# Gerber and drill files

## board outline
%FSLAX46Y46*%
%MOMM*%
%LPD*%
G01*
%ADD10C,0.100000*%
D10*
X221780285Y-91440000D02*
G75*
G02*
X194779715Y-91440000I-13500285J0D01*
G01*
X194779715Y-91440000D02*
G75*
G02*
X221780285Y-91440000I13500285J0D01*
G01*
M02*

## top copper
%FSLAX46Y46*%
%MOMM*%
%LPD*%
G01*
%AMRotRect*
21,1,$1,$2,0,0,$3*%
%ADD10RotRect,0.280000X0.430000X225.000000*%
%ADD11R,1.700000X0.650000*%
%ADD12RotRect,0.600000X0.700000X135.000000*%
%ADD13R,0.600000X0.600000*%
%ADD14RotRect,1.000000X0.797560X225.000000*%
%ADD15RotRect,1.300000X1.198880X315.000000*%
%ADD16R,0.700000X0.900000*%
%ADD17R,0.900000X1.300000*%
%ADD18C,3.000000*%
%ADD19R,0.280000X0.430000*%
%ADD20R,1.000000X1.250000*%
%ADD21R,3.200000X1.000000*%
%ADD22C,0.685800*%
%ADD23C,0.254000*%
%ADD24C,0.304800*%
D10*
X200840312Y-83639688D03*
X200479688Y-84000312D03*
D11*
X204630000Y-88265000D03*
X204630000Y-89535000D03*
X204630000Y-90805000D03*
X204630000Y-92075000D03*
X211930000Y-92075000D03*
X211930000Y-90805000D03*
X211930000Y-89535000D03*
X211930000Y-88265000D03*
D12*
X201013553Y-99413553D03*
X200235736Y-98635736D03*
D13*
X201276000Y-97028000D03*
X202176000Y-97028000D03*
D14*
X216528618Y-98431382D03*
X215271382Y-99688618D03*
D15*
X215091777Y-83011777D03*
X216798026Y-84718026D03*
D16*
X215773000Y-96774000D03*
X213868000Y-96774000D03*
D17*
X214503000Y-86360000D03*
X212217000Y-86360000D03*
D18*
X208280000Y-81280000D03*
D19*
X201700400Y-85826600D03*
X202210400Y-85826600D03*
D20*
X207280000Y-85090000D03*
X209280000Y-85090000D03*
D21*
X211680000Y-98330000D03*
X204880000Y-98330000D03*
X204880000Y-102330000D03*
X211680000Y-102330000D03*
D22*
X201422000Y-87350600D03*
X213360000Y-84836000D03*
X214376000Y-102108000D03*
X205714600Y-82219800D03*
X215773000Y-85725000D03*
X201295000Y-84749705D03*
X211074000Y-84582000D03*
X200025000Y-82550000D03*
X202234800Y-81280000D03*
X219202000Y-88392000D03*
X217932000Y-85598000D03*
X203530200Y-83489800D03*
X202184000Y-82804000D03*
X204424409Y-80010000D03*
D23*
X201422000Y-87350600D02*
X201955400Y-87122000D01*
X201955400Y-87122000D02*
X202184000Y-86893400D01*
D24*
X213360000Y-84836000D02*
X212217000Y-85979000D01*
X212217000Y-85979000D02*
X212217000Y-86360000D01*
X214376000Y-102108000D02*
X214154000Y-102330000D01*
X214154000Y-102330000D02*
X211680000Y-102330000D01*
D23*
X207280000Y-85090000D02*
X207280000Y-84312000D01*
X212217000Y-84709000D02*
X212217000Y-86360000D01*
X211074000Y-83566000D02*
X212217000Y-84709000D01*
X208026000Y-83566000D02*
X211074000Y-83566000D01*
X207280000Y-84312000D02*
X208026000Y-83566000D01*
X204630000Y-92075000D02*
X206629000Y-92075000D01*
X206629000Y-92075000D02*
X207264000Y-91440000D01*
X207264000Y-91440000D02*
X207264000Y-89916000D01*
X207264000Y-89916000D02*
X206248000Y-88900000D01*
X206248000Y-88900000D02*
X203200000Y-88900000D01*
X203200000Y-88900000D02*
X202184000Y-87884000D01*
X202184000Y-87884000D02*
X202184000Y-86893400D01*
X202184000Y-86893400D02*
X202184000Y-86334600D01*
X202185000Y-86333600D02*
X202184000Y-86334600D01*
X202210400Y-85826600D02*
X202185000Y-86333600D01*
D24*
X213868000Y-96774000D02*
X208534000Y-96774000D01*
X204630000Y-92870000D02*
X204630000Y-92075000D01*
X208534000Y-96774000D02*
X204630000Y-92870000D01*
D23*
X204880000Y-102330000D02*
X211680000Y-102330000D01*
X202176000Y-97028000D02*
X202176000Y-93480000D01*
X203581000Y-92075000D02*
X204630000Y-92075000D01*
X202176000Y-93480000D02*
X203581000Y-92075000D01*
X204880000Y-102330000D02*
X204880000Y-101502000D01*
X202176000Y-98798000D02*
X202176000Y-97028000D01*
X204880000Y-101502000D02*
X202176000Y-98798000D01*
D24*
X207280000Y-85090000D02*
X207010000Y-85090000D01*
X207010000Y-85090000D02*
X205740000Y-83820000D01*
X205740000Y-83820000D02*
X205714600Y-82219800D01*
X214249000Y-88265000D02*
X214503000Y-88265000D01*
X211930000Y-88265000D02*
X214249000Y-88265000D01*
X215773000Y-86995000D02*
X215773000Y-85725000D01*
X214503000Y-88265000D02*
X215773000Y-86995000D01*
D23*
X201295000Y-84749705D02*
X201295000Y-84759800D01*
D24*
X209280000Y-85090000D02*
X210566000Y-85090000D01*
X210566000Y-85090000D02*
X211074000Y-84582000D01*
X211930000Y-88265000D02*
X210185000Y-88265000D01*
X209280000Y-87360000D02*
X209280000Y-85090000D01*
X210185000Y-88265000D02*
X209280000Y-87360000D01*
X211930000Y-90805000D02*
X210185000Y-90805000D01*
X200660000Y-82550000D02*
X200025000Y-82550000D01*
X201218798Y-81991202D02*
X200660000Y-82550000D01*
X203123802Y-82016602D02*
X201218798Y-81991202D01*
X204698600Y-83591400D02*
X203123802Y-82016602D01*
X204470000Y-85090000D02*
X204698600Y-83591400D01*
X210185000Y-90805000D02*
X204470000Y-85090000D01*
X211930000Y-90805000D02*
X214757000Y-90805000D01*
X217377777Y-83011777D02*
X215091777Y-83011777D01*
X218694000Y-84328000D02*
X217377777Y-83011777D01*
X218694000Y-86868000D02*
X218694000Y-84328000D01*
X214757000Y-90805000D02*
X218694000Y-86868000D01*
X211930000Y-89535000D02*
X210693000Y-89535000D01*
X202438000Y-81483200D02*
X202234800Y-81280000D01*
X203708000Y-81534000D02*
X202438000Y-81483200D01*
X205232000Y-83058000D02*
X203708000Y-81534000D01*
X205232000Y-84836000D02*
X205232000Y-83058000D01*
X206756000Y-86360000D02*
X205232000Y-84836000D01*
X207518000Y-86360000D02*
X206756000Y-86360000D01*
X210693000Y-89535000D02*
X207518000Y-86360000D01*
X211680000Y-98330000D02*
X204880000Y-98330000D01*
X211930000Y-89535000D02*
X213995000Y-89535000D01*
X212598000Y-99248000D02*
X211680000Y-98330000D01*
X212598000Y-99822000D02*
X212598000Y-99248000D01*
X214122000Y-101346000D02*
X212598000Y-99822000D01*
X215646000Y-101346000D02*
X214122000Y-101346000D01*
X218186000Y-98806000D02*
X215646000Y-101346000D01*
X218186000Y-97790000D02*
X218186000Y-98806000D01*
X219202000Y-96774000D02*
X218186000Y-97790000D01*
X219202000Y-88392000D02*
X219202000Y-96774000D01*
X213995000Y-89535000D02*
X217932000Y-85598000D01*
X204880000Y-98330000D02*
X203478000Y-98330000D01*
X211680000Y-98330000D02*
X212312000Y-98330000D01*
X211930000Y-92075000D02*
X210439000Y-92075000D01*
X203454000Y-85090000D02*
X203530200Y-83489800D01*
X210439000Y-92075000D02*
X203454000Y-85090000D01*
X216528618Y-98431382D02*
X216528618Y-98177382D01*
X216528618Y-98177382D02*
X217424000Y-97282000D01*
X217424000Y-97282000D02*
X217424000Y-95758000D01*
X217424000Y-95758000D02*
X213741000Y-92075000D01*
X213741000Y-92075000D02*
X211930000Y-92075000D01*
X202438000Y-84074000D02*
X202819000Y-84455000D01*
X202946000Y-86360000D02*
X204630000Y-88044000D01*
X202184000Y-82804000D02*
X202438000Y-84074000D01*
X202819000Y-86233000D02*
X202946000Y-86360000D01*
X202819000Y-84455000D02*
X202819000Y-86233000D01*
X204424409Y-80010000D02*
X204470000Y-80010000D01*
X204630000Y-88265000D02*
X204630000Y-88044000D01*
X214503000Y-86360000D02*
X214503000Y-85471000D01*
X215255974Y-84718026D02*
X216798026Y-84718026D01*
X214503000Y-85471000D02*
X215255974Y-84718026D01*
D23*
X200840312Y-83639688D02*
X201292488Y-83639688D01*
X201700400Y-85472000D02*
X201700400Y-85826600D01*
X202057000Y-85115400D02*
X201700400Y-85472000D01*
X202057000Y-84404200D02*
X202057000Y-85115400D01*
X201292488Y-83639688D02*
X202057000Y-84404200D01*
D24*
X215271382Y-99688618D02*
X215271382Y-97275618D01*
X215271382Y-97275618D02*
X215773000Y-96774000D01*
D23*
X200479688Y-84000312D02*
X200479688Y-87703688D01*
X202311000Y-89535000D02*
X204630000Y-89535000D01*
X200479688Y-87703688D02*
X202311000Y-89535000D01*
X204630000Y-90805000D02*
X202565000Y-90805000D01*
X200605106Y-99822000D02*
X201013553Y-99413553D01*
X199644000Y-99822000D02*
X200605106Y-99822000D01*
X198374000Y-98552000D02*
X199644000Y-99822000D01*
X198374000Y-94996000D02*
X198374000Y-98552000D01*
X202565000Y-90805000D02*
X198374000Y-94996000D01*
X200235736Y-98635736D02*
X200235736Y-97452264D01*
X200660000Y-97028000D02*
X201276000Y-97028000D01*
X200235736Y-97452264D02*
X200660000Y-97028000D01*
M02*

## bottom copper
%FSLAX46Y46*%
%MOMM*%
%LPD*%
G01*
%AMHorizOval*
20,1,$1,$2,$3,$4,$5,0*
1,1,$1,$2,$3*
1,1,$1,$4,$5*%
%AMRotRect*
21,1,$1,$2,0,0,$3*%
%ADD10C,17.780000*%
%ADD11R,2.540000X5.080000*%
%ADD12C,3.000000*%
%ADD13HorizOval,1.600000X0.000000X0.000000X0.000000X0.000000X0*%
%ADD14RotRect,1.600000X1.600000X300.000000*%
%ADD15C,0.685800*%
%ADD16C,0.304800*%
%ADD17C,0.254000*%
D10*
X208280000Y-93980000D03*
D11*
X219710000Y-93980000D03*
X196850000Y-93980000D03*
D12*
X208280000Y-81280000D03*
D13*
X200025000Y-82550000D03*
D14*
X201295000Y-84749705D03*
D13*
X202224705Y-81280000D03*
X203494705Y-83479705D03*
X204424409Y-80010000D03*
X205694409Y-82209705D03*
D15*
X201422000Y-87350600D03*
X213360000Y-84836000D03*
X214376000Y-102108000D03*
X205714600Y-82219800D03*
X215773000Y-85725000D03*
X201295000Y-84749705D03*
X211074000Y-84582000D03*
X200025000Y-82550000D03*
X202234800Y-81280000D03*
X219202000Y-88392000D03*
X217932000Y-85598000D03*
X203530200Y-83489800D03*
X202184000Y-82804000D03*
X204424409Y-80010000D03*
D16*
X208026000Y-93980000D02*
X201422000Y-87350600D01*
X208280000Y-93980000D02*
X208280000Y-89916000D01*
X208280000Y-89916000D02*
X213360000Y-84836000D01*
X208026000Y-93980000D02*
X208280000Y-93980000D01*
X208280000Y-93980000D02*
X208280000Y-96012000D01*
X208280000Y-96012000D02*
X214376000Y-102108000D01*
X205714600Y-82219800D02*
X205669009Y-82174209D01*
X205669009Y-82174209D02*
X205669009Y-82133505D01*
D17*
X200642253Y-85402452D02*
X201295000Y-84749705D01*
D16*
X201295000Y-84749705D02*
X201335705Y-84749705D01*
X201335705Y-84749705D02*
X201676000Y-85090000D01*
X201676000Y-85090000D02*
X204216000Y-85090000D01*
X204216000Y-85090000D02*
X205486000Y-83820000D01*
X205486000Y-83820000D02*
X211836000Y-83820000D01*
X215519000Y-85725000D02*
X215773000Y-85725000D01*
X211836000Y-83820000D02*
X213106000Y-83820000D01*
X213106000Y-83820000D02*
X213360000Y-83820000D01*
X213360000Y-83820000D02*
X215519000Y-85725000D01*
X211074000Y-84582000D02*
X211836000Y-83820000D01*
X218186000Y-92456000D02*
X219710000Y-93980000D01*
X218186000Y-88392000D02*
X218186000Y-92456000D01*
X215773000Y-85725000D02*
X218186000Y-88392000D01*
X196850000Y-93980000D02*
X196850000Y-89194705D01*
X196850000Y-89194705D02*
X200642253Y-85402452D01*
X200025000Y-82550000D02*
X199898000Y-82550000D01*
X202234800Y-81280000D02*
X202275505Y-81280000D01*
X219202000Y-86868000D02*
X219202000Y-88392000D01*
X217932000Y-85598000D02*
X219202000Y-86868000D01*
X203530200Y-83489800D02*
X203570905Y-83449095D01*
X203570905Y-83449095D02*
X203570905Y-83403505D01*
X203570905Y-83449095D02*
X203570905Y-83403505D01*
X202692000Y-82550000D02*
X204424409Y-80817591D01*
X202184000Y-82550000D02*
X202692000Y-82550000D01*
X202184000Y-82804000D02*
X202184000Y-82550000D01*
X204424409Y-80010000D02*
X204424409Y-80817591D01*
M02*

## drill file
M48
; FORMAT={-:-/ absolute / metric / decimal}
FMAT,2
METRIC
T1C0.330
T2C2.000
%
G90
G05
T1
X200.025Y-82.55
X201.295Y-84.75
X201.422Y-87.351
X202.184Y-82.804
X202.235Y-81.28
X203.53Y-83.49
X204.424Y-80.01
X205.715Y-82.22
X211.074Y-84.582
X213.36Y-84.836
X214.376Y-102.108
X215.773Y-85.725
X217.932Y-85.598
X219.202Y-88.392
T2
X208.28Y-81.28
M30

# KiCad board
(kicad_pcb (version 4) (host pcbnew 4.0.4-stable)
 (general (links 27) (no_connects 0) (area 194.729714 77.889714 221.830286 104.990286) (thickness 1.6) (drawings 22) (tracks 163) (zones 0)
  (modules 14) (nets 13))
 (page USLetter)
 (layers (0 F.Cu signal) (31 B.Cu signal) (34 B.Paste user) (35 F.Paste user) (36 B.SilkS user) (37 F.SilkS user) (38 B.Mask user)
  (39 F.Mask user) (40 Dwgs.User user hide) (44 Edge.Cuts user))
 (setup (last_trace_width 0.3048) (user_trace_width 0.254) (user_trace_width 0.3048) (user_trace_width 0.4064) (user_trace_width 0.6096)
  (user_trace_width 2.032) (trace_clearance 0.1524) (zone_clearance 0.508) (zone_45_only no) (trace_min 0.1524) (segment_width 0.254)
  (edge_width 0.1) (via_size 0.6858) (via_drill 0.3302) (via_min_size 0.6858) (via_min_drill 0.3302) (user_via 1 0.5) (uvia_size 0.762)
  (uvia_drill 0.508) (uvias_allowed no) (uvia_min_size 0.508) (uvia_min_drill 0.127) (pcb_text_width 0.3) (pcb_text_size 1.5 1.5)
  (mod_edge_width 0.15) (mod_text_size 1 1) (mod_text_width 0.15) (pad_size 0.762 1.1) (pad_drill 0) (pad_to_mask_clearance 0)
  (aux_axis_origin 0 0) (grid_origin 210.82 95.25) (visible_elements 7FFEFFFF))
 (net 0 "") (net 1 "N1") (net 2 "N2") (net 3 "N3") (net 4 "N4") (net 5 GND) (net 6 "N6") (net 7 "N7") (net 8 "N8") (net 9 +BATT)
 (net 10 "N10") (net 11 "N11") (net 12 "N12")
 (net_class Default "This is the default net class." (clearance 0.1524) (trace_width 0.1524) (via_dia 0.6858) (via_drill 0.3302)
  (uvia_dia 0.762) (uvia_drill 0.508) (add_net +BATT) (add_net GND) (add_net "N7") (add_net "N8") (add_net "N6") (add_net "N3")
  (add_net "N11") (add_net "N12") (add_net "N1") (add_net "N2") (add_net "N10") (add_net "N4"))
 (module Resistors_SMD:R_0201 (layer F.Cu) (at 200.66 83.82 225)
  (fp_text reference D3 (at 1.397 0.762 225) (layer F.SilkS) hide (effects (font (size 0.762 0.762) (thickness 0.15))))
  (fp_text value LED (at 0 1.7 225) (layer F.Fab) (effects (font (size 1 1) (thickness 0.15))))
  (pad 1 smd rect (at -0.255 0 225) (size 0.28 0.43) (layers F.Cu F.Paste F.Mask) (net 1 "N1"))
  (pad 2 smd rect (at 0.255 0 225) (size 0.28 0.43) (layers F.Cu F.Paste F.Mask) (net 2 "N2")))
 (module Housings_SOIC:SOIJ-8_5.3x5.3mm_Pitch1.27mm (layer F.Cu) (at 208.28 90.17)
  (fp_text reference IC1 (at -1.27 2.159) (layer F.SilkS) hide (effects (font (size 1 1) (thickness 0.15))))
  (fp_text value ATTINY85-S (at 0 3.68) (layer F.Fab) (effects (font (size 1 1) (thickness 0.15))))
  (pad 1 smd rect (at -3.65 -1.905) (size 1.7 0.65) (layers F.Cu F.Paste F.Mask) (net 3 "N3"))
  (pad 2 smd rect (at -3.65 -0.635) (size 1.7 0.65) (layers F.Cu F.Paste F.Mask) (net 2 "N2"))
  (pad 3 smd rect (at -3.65 0.635) (size 1.7 0.65) (layers F.Cu F.Paste F.Mask) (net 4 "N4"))
  (pad 4 smd rect (at -3.65 1.905) (size 1.7 0.65) (layers F.Cu F.Paste F.Mask) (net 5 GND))
  (pad 5 smd rect (at 3.65 1.905) (size 1.7 0.65) (layers F.Cu F.Paste F.Mask) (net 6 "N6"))
  (pad 6 smd rect (at 3.65 0.635) (size 1.7 0.65) (layers F.Cu F.Paste F.Mask) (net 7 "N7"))
  (pad 7 smd rect (at 3.65 -0.635) (size 1.7 0.65) (layers F.Cu F.Paste F.Mask) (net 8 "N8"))
  (pad 8 smd rect (at 3.65 -1.905) (size 1.7 0.65) (layers F.Cu F.Paste F.Mask) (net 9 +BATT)))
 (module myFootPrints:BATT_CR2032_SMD (layer B.Cu) (at 208.28 93.98 180)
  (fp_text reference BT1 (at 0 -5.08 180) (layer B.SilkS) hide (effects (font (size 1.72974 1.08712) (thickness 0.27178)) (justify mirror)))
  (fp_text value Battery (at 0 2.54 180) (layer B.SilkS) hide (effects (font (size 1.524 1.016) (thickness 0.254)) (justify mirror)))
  (pad 2 smd circle (at 0 0 180) (size 17.78 17.78) (layers B.Cu B.Paste B.Mask) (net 5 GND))
  (pad 1 smd rect (at -11.43 0 180) (size 2.54 5.08) (layers B.Cu B.Paste B.Mask) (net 9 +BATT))
  (pad 1 smd rect (at 11.43 0 180) (size 2.54 5.08) (layers B.Cu B.Paste B.Mask) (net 9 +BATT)))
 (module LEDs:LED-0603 (layer F.Cu) (at 200.66 99.06 315)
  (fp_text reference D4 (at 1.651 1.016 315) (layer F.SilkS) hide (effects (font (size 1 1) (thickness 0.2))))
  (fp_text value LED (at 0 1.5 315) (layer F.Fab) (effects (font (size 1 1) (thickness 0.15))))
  (pad 2 smd rect (at 0.5 0 135) (size 0.6 0.7) (layers F.Cu F.Paste F.Mask) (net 4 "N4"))
  (pad 1 smd rect (at -0.6 0 135) (size 0.6 0.7) (layers F.Cu F.Paste F.Mask) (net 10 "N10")))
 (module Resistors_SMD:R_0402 (layer F.Cu) (at 201.676 97.028)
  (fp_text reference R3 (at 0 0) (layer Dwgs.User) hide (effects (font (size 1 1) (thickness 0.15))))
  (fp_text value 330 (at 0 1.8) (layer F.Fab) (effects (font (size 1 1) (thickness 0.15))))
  (pad 1 smd rect (at -0.4 0) (size 0.6 0.6) (layers F.Cu F.Paste F.Mask) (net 10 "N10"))
  (pad 2 smd rect (at 0.5 0) (size 0.6 0.6) (layers F.Cu F.Paste F.Mask) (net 5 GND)))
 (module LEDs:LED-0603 (layer F.Cu) (at 215.9 99.06 45)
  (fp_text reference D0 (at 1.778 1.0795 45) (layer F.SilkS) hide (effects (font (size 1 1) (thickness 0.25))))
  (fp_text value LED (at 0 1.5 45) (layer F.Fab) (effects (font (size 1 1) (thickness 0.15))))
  (pad 2 smd rect (at 0.889 0 225) (size 1 0.79756) (layers F.Cu F.Paste F.Mask) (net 6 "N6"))
  (pad 1 smd rect (at -0.889 0 225) (size 1 0.79756) (layers F.Cu F.Paste F.Mask) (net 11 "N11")))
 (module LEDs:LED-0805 (layer F.Cu) (at 215.9 83.82 135)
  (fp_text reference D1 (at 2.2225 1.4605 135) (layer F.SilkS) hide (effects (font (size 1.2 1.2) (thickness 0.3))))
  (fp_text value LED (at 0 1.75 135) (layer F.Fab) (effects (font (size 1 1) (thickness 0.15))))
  (pad 2 smd rect (at 1.143 0 315) (size 1.3 1.19888) (layers F.Cu F.Paste F.Mask) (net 7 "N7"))
  (pad 1 smd rect (at -1.27 0 315) (size 1.3 1.19888) (layers F.Cu F.Paste F.Mask) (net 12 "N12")))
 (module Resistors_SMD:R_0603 (layer F.Cu) (at 214.884 96.774 180)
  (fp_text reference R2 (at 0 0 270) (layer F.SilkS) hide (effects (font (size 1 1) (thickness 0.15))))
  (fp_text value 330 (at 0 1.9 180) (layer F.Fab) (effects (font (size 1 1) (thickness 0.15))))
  (pad 1 smd rect (at -0.889 0 180) (size 0.7 0.9) (layers F.Cu F.Paste F.Mask) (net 11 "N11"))
  (pad 2 smd rect (at 1.016 0 180) (size 0.7 0.9) (layers F.Cu F.Paste F.Mask) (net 5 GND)))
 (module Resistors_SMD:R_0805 (layer F.Cu) (at 213.36 86.36 180)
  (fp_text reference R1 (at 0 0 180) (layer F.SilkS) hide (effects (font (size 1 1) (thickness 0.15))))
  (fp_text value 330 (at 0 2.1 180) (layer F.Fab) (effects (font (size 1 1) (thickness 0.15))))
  (pad 1 smd rect (at -1.143 0 180) (size 0.9 1.3) (layers F.Cu F.Paste F.Mask) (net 12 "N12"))
  (pad 2 smd rect (at 1.143 0 180) (size 0.9 1.3) (layers F.Cu F.Paste F.Mask) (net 5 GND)))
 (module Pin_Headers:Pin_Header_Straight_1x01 (layer F.Cu) (at 208.28 81.28)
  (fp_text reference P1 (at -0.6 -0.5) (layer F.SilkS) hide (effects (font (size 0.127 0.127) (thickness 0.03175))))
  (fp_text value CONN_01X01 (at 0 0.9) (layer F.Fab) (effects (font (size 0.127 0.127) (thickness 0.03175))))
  (pad P5 thru_hole circle (at 0 0) (size 3 3) (drill 2) (layers *.Cu *.Mask)))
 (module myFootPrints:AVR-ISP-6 (layer B.Cu) (at 200.025 82.55 300)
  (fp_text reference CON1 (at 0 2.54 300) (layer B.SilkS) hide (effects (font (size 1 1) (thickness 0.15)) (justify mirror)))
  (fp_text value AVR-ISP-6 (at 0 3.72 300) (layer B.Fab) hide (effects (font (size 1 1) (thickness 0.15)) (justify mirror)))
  (pad 1 smd oval (at 0 0 300) (size 1.6 1.6) (layers B.Cu B.Paste B.Mask) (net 7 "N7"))
  (pad 2 smd rect (at 2.54 0 300) (size 1.6 1.6) (layers B.Cu B.Paste B.Mask) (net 9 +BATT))
  (pad 3 smd oval (at 0 -2.54 300) (size 1.6 1.6) (layers B.Cu B.Paste B.Mask) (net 8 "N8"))
  (pad 4 smd oval (at 2.54 -2.54 300) (size 1.6 1.6) (layers B.Cu B.Paste B.Mask) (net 6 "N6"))
  (pad 5 smd oval (at 0 -5.08 300) (size 1.6 1.6) (layers B.Cu B.Paste B.Mask) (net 3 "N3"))
  (pad 6 smd oval (at 2.54 -5.08 300) (size 1.6 1.6) (layers B.Cu B.Paste B.Mask) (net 5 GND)))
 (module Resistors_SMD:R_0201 (layer F.Cu) (at 201.9554 85.8266)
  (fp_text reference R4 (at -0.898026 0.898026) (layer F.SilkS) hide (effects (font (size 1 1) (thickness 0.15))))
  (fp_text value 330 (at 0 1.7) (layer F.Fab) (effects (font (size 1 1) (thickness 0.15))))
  (pad 1 smd rect (at -0.255 0) (size 0.28 0.43) (layers F.Cu F.Paste F.Mask) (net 1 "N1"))
  (pad 2 smd rect (at 0.255 0) (size 0.28 0.43) (layers F.Cu F.Paste F.Mask) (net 5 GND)))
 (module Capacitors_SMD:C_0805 (layer F.Cu) (at 208.28 85.09)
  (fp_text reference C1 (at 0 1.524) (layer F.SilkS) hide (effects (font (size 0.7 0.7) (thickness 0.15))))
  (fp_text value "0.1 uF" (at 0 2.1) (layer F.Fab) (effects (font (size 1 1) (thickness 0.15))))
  (pad 1 smd rect (at -1 0) (size 1 1.25) (layers F.Cu F.Paste F.Mask) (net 5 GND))
  (pad 2 smd rect (at 1 0) (size 1 1.25) (layers F.Cu F.Paste F.Mask) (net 9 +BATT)))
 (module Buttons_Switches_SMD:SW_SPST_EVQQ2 (layer F.Cu) (at 208.28 100.33)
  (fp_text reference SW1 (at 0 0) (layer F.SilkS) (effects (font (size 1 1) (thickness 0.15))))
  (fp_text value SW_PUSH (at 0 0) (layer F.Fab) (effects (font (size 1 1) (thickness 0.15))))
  (pad 1 smd rect (at 3.4 -2) (size 3.2 1) (layers F.Cu F.Paste F.Mask) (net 8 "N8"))
  (pad 1 smd rect (at -3.4 -2) (size 3.2 1) (layers F.Cu F.Paste F.Mask) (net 8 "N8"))
  (pad 2 smd rect (at -3.4 2) (size 3.2 1) (layers F.Cu F.Paste F.Mask) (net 5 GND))
  (pad 2 smd rect (at 3.4 2) (size 3.2 1) (layers F.Cu F.Paste F.Mask) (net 5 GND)))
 (gr_circle (center 208.28 91.44) (end 198.12 82.55) (layer Edge.Cuts) (width 0.1))
 (segment (start 201.422 87.3506) (end 201.9554 87.122) (width 0.254) (layer F.Cu) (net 5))
 (segment (start 208.026 93.98) (end 201.422 87.3506) (width 0.3048) (layer B.Cu) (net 5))
 (via (at 201.422 87.3506) (size 0.6858) (drill 0.3302) (layers F.Cu B.Cu) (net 5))
 (segment (start 201.9554 87.122) (end 202.184 86.8934) (width 0.254) (layer F.Cu) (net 5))
 (segment (start 208.28 93.98) (end 208.28 89.916) (width 0.3048) (layer B.Cu) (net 5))
 (segment (start 208.28 89.916) (end 213.36 84.836) (width 0.3048) (layer B.Cu) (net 5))
 (segment (start 213.36 84.836) (end 212.217 85.979) (width 0.3048) (layer F.Cu) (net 5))
 (via (at 213.36 84.836) (size 0.6858) (drill 0.3302) (layers F.Cu B.Cu) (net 5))
 (segment (start 212.217 85.979) (end 212.217 86.36) (width 0.3048) (layer F.Cu) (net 5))
 (segment (start 208.026 93.98) (end 208.28 93.98) (width 0.3048) (layer B.Cu) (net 5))
 (segment (start 208.28 93.98) (end 208.28 96.012) (width 0.3048) (layer B.Cu) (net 5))
 (segment (start 208.28 96.012) (end 214.376 102.108) (width 0.3048) (layer B.Cu) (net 5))
 (via (at 214.376 102.108) (size 0.6858) (drill 0.3302) (layers F.Cu B.Cu) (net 5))
 (segment (start 214.376 102.108) (end 214.154 102.33) (width 0.3048) (layer F.Cu) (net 5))
 (segment (start 214.154 102.33) (end 211.68 102.33) (width 0.3048) (layer F.Cu) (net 5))
 (segment (start 207.28 85.09) (end 207.28 84.312) (width 0.254) (layer F.Cu) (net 5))
 (segment (start 212.217 84.709) (end 212.217 86.36) (width 0.254) (layer F.Cu) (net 5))
 (segment (start 211.074 83.566) (end 212.217 84.709) (width 0.254) (layer F.Cu) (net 5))
 (segment (start 208.026 83.566) (end 211.074 83.566) (width 0.254) (layer F.Cu) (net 5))
 (segment (start 207.28 84.312) (end 208.026 83.566) (width 0.254) (layer F.Cu) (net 5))
 (segment (start 204.63 92.075) (end 206.629 92.075) (width 0.254) (layer F.Cu) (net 5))
 (segment (start 206.629 92.075) (end 207.264 91.44) (width 0.254) (layer F.Cu) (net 5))
 (segment (start 207.264 91.44) (end 207.264 89.916) (width 0.254) (layer F.Cu) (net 5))
 (segment (start 207.264 89.916) (end 206.248 88.9) (width 0.254) (layer F.Cu) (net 5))
 (segment (start 206.248 88.9) (end 203.2 88.9) (width 0.254) (layer F.Cu) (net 5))
 (segment (start 203.2 88.9) (end 202.184 87.884) (width 0.254) (layer F.Cu) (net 5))
 (segment (start 202.184 87.884) (end 202.184 86.8934) (width 0.254) (layer F.Cu) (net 5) (status 20))
 (segment (start 202.184 86.8934) (end 202.184 86.3346) (width 0.254) (layer F.Cu) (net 5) (status 20))
 (segment (start 202.185 86.3336) (end 202.184 86.3346) (width 0.254) (layer F.Cu) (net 5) (status 30))
 (segment (start 202.2104 85.8266) (end 202.185 86.3336) (width 0.254) (layer F.Cu) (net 5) (status 10))
 (segment (start 213.868 96.774) (end 208.534 96.774) (width 0.3048) (layer F.Cu) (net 5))
 (segment (start 204.63 92.87) (end 204.63 92.075) (width 0.3048) (layer F.Cu) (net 5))
 (segment (start 208.534 96.774) (end 204.63 92.87) (width 0.3048) (layer F.Cu) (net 5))
 (segment (start 204.88 102.33) (end 211.68 102.33) (width 0.254) (layer F.Cu) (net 5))
 (segment (start 202.176 97.028) (end 202.176 93.48) (width 0.254) (layer F.Cu) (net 5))
 (segment (start 203.581 92.075) (end 204.63 92.075) (width 0.254) (layer F.Cu) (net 5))
 (segment (start 202.176 93.48) (end 203.581 92.075) (width 0.254) (layer F.Cu) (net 5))
 (segment (start 204.88 102.33) (end 204.88 101.502) (width 0.254) (layer F.Cu) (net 5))
 (segment (start 202.176 98.798) (end 202.176 97.028) (width 0.254) (layer F.Cu) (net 5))
 (segment (start 204.88 101.502) (end 202.176 98.798) (width 0.254) (layer F.Cu) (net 5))
 (segment (start 207.28 85.09) (end 207.01 85.09) (width 0.3048) (layer F.Cu) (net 5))
 (segment (start 207.01 85.09) (end 205.74 83.82) (width 0.3048) (layer F.Cu) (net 5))
 (segment (start 205.74 83.82) (end 205.7146 82.2198) (width 0.3048) (layer F.Cu) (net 5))
 (via (at 205.7146 82.2198) (size 0.6858) (drill 0.3302) (layers F.Cu B.Cu) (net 5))
 (segment (start 205.7146 82.2198) (end 205.669009 82.174209) (width 0.3048) (layer B.Cu) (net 5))
 (segment (start 205.669009 82.174209) (end 205.669009 82.133505) (width 0.3048) (layer B.Cu) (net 5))
 (segment (start 214.249 88.265) (end 214.503 88.265) (width 0.3048) (layer F.Cu) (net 9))
 (via (at 215.773 85.725) (size 0.6858) (drill 0.3302) (layers F.Cu B.Cu) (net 9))
 (segment (start 211.93 88.265) (end 214.249 88.265) (width 0.3048) (layer F.Cu) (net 9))
 (segment (start 215.773 86.995) (end 215.773 85.725) (width 0.3048) (layer F.Cu) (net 9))
 (segment (start 214.503 88.265) (end 215.773 86.995) (width 0.3048) (layer F.Cu) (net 9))
 (via (at 201.295 84.749705) (size 0.6858) (drill 0.3302) (layers F.Cu B.Cu) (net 9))
 (segment (start 201.295 84.749705) (end 201.295 84.7598) (width 0.254) (layer F.Cu) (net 9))
 (segment (start 200.642253 85.402452) (end 201.295 84.749705) (width 0.254) (layer B.Cu) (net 9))
 (segment (start 201.295 84.749705) (end 201.335705 84.749705) (width 0.3048) (layer B.Cu) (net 9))
 (segment (start 201.335705 84.749705) (end 201.676 85.09) (width 0.3048) (layer B.Cu) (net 9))
 (segment (start 201.676 85.09) (end 204.216 85.09) (width 0.3048) (layer B.Cu) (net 9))
 (segment (start 204.216 85.09) (end 205.486 83.82) (width 0.3048) (layer B.Cu) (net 9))
 (segment (start 205.486 83.82) (end 211.836 83.82) (width 0.3048) (layer B.Cu) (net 9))
 (segment (start 209.28 85.09) (end 210.566 85.09) (width 0.3048) (layer F.Cu) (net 9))
 (segment (start 215.519 85.725) (end 215.773 85.725) (width 0.3048) (layer B.Cu) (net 9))
 (segment (start 211.836 83.82) (end 213.106 83.82) (width 0.3048) (layer B.Cu) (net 9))
 (segment (start 213.106 83.82) (end 213.36 83.82) (width 0.3048) (layer B.Cu) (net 9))
 (segment (start 213.36 83.82) (end 215.519 85.725) (width 0.3048) (layer B.Cu) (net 9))
 (segment (start 211.074 84.582) (end 211.836 83.82) (width 0.3048) (layer B.Cu) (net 9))
 (via (at 211.074 84.582) (size 0.6858) (drill 0.3302) (layers F.Cu B.Cu) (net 9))
 (segment (start 210.566 85.09) (end 211.074 84.582) (width 0.3048) (layer F.Cu) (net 9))
 (segment (start 218.186 92.456) (end 219.71 93.98) (width 0.3048) (layer B.Cu) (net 9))
 (segment (start 218.186 88.392) (end 218.186 92.456) (width 0.3048) (layer B.Cu) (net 9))
 (segment (start 215.773 85.725) (end 218.186 88.392) (width 0.3048) (layer B.Cu) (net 9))
 (segment (start 196.85 93.98) (end 196.85 89.194705) (width 0.3048) (layer B.Cu) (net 9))
 (segment (start 196.85 89.194705) (end 200.642253 85.402452) (width 0.3048) (layer B.Cu) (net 9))
 (segment (start 211.93 88.265) (end 210.185 88.265) (width 0.3048) (layer F.Cu) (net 9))
 (segment (start 209.28 87.36) (end 209.28 85.09) (width 0.3048) (layer F.Cu) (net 9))
 (segment (start 210.185 88.265) (end 209.28 87.36) (width 0.3048) (layer F.Cu) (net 9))
 (segment (start 211.93 90.805) (end 210.185 90.805) (width 0.3048) (layer F.Cu) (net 7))
 (segment (start 200.025 82.55) (end 199.898 82.55) (width 0.3048) (layer B.Cu) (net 7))
 (via (at 200.025 82.55) (size 0.6858) (drill 0.3302) (layers F.Cu B.Cu) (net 7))
 (segment (start 200.66 82.55) (end 200.025 82.55) (width 0.3048) (layer F.Cu) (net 7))
 (segment (start 201.218798 81.991202) (end 200.66 82.55) (width 0.3048) (layer F.Cu) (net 7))
 (segment (start 203.123802 82.016602) (end 201.218798 81.991202) (width 0.3048) (layer F.Cu) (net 7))
 (segment (start 204.6986 83.5914) (end 203.123802 82.016602) (width 0.3048) (layer F.Cu) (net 7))
 (segment (start 204.47 85.09) (end 204.6986 83.5914) (width 0.3048) (layer F.Cu) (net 7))
 (segment (start 210.185 90.805) (end 204.47 85.09) (width 0.3048) (layer F.Cu) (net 7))
 (segment (start 211.93 90.805) (end 214.757 90.805) (width 0.3048) (layer F.Cu) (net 7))
 (segment (start 217.377777 83.011777) (end 215.091777 83.011777) (width 0.3048) (layer F.Cu) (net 7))
 (segment (start 218.694 84.328) (end 217.377777 83.011777) (width 0.3048) (layer F.Cu) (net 7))
 (segment (start 218.694 86.868) (end 218.694 84.328) (width 0.3048) (layer F.Cu) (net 7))
 (segment (start 214.757 90.805) (end 218.694 86.868) (width 0.3048) (layer F.Cu) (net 7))
 (segment (start 211.93 89.535) (end 210.693 89.535) (width 0.3048) (layer F.Cu) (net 8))
 (segment (start 202.2348 81.28) (end 202.275505 81.28) (width 0.3048) (layer B.Cu) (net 8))
 (via (at 202.2348 81.28) (size 0.6858) (drill 0.3302) (layers F.Cu B.Cu) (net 8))
 (segment (start 202.438 81.4832) (end 202.2348 81.28) (width 0.3048) (layer F.Cu) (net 8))
 (segment (start 203.708 81.534) (end 202.438 81.4832) (width 0.3048) (layer F.Cu) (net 8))
 (segment (start 205.232 83.058) (end 203.708 81.534) (width 0.3048) (layer F.Cu) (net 8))
 (segment (start 205.232 84.836) (end 205.232 83.058) (width 0.3048) (layer F.Cu) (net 8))
 (segment (start 206.756 86.36) (end 205.232 84.836) (width 0.3048) (layer F.Cu) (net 8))
 (segment (start 207.518 86.36) (end 206.756 86.36) (width 0.3048) (layer F.Cu) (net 8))
 (segment (start 210.693 89.535) (end 207.518 86.36) (width 0.3048) (layer F.Cu) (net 8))
 (segment (start 211.68 98.33) (end 204.88 98.33) (width 0.3048) (layer F.Cu) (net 8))
 (segment (start 211.93 89.535) (end 213.995 89.535) (width 0.3048) (layer F.Cu) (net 8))
 (segment (start 212.598 99.248) (end 211.68 98.33) (width 0.3048) (layer F.Cu) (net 8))
 (segment (start 212.598 99.822) (end 212.598 99.248) (width 0.3048) (layer F.Cu) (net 8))
 (segment (start 214.122 101.346) (end 212.598 99.822) (width 0.3048) (layer F.Cu) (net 8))
 (segment (start 215.646 101.346) (end 214.122 101.346) (width 0.3048) (layer F.Cu) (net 8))
 (segment (start 218.186 98.806) (end 215.646 101.346) (width 0.3048) (layer F.Cu) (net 8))
 (segment (start 218.186 97.79) (end 218.186 98.806) (width 0.3048) (layer F.Cu) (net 8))
 (segment (start 219.202 96.774) (end 218.186 97.79) (width 0.3048) (layer F.Cu) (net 8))
 (segment (start 219.202 88.392) (end 219.202 96.774) (width 0.3048) (layer F.Cu) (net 8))
 (via (at 219.202 88.392) (size 0.6858) (drill 0.3302) (layers F.Cu B.Cu) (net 8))
 (segment (start 219.202 86.868) (end 219.202 88.392) (width 0.3048) (layer B.Cu) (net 8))
 (segment (start 217.932 85.598) (end 219.202 86.868) (width 0.3048) (layer B.Cu) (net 8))
 (via (at 217.932 85.598) (size 0.6858) (drill 0.3302) (layers F.Cu B.Cu) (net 8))
 (segment (start 213.995 89.535) (end 217.932 85.598) (width 0.3048) (layer F.Cu) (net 8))
 (segment (start 204.88 98.33) (end 203.478 98.33) (width 0.3048) (layer F.Cu) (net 8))
 (segment (start 211.68 98.33) (end 212.312 98.33) (width 0.3048) (layer F.Cu) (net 8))
 (segment (start 211.93 92.075) (end 210.439 92.075) (width 0.3048) (layer F.Cu) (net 6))
 (segment (start 203.5302 83.4898) (end 203.570905 83.449095) (width 0.3048) (layer B.Cu) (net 6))
 (via (at 203.5302 83.4898) (size 0.6858) (drill 0.3302) (layers F.Cu B.Cu) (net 6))
 (segment (start 203.454 85.09) (end 203.5302 83.4898) (width 0.3048) (layer F.Cu) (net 6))
 (segment (start 210.439 92.075) (end 203.454 85.09) (width 0.3048) (layer F.Cu) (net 6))
 (segment (start 203.570905 83.449095) (end 203.570905 83.403505) (width 0.3048) (layer B.Cu) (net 6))
 (segment (start 203.570905 83.449095) (end 203.570905 83.403505) (width 0.3048) (layer B.Cu) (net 6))
 (segment (start 216.528618 98.431382) (end 216.528618 98.177382) (width 0.3048) (layer F.Cu) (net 6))
 (segment (start 216.528618 98.177382) (end 217.424 97.282) (width 0.3048) (layer F.Cu) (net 6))
 (segment (start 217.424 97.282) (end 217.424 95.758) (width 0.3048) (layer F.Cu) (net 6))
 (segment (start 217.424 95.758) (end 213.741 92.075) (width 0.3048) (layer F.Cu) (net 6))
 (segment (start 213.741 92.075) (end 211.93 92.075) (width 0.3048) (layer F.Cu) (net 6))
 (segment (start 202.438 84.074) (end 202.819 84.455) (width 0.3048) (layer F.Cu) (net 3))
 (segment (start 202.692 82.55) (end 204.424409 80.817591) (width 0.3048) (layer B.Cu) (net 3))
 (segment (start 202.184 82.55) (end 202.692 82.55) (width 0.3048) (layer B.Cu) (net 3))
 (segment (start 202.184 82.804) (end 202.184 82.55) (width 0.3048) (layer B.Cu) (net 3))
 (via (at 202.184 82.804) (size 0.6858) (drill 0.3302) (layers F.Cu B.Cu) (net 3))
 (segment (start 204.424409 80.01) (end 204.424409 80.817591) (width 0.3048) (layer B.Cu) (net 3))
 (segment (start 202.946 86.36) (end 204.63 88.044) (width 0.3048) (layer F.Cu) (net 3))
 (segment (start 202.184 82.804) (end 202.438 84.074) (width 0.3048) (layer F.Cu) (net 3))
 (segment (start 202.819 86.233) (end 202.946 86.36) (width 0.3048) (layer F.Cu) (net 3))
 (segment (start 202.819 84.455) (end 202.819 86.233) (width 0.3048) (layer F.Cu) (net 3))
 (via (at 204.424409 80.01) (size 0.6858) (drill 0.3302) (layers F.Cu B.Cu) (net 3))
 (segment (start 204.424409 80.01) (end 204.47 80.01) (width 0.3048) (layer F.Cu) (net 3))
 (segment (start 204.63 88.265) (end 204.63 88.044) (width 0.3048) (layer F.Cu) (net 3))
 (segment (start 214.503 86.36) (end 214.503 85.471) (width 0.3048) (layer F.Cu) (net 12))
 (segment (start 215.255974 84.718026) (end 216.798026 84.718026) (width 0.3048) (layer F.Cu) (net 12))
 (segment (start 214.503 85.471) (end 215.255974 84.718026) (width 0.3048) (layer F.Cu) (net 12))
 (segment (start 200.840312 83.639688) (end 201.292488 83.639688) (width 0.254) (layer F.Cu) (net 1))
 (segment (start 201.7004 85.472) (end 201.7004 85.8266) (width 0.254) (layer F.Cu) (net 1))
 (segment (start 202.057 85.1154) (end 201.7004 85.472) (width 0.254) (layer F.Cu) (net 1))
 (segment (start 202.057 84.4042) (end 202.057 85.1154) (width 0.254) (layer F.Cu) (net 1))
 (segment (start 201.292488 83.639688) (end 202.057 84.4042) (width 0.254) (layer F.Cu) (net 1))
 (segment (start 215.271382 99.688618) (end 215.271382 97.275618) (width 0.3048) (layer F.Cu) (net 11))
 (segment (start 215.271382 97.275618) (end 215.773 96.774) (width 0.3048) (layer F.Cu) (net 11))
 (segment (start 200.479688 84.000312) (end 200.479688 87.703688) (width 0.254) (layer F.Cu) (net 2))
 (segment (start 202.311 89.535) (end 204.63 89.535) (width 0.254) (layer F.Cu) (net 2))
 (segment (start 200.479688 87.703688) (end 202.311 89.535) (width 0.254) (layer F.Cu) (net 2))
 (segment (start 204.63 90.805) (end 202.565 90.805) (width 0.254) (layer F.Cu) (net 4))
 (segment (start 200.605106 99.822) (end 201.013553 99.413553) (width 0.254) (layer F.Cu) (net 4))
 (segment (start 199.644 99.822) (end 200.605106 99.822) (width 0.254) (layer F.Cu) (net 4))
 (segment (start 198.374 98.552) (end 199.644 99.822) (width 0.254) (layer F.Cu) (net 4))
 (segment (start 198.374 94.996) (end 198.374 98.552) (width 0.254) (layer F.Cu) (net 4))
 (segment (start 202.565 90.805) (end 198.374 94.996) (width 0.254) (layer F.Cu) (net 4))
 (segment (start 200.235736 98.635736) (end 200.235736 97.452264) (width 0.254) (layer F.Cu) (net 10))
 (segment (start 200.66 97.028) (end 201.276 97.028) (width 0.254) (layer F.Cu) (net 10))
 (segment (start 200.235736 97.452264) (end 200.66 97.028) (width 0.254) (layer F.Cu) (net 10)))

